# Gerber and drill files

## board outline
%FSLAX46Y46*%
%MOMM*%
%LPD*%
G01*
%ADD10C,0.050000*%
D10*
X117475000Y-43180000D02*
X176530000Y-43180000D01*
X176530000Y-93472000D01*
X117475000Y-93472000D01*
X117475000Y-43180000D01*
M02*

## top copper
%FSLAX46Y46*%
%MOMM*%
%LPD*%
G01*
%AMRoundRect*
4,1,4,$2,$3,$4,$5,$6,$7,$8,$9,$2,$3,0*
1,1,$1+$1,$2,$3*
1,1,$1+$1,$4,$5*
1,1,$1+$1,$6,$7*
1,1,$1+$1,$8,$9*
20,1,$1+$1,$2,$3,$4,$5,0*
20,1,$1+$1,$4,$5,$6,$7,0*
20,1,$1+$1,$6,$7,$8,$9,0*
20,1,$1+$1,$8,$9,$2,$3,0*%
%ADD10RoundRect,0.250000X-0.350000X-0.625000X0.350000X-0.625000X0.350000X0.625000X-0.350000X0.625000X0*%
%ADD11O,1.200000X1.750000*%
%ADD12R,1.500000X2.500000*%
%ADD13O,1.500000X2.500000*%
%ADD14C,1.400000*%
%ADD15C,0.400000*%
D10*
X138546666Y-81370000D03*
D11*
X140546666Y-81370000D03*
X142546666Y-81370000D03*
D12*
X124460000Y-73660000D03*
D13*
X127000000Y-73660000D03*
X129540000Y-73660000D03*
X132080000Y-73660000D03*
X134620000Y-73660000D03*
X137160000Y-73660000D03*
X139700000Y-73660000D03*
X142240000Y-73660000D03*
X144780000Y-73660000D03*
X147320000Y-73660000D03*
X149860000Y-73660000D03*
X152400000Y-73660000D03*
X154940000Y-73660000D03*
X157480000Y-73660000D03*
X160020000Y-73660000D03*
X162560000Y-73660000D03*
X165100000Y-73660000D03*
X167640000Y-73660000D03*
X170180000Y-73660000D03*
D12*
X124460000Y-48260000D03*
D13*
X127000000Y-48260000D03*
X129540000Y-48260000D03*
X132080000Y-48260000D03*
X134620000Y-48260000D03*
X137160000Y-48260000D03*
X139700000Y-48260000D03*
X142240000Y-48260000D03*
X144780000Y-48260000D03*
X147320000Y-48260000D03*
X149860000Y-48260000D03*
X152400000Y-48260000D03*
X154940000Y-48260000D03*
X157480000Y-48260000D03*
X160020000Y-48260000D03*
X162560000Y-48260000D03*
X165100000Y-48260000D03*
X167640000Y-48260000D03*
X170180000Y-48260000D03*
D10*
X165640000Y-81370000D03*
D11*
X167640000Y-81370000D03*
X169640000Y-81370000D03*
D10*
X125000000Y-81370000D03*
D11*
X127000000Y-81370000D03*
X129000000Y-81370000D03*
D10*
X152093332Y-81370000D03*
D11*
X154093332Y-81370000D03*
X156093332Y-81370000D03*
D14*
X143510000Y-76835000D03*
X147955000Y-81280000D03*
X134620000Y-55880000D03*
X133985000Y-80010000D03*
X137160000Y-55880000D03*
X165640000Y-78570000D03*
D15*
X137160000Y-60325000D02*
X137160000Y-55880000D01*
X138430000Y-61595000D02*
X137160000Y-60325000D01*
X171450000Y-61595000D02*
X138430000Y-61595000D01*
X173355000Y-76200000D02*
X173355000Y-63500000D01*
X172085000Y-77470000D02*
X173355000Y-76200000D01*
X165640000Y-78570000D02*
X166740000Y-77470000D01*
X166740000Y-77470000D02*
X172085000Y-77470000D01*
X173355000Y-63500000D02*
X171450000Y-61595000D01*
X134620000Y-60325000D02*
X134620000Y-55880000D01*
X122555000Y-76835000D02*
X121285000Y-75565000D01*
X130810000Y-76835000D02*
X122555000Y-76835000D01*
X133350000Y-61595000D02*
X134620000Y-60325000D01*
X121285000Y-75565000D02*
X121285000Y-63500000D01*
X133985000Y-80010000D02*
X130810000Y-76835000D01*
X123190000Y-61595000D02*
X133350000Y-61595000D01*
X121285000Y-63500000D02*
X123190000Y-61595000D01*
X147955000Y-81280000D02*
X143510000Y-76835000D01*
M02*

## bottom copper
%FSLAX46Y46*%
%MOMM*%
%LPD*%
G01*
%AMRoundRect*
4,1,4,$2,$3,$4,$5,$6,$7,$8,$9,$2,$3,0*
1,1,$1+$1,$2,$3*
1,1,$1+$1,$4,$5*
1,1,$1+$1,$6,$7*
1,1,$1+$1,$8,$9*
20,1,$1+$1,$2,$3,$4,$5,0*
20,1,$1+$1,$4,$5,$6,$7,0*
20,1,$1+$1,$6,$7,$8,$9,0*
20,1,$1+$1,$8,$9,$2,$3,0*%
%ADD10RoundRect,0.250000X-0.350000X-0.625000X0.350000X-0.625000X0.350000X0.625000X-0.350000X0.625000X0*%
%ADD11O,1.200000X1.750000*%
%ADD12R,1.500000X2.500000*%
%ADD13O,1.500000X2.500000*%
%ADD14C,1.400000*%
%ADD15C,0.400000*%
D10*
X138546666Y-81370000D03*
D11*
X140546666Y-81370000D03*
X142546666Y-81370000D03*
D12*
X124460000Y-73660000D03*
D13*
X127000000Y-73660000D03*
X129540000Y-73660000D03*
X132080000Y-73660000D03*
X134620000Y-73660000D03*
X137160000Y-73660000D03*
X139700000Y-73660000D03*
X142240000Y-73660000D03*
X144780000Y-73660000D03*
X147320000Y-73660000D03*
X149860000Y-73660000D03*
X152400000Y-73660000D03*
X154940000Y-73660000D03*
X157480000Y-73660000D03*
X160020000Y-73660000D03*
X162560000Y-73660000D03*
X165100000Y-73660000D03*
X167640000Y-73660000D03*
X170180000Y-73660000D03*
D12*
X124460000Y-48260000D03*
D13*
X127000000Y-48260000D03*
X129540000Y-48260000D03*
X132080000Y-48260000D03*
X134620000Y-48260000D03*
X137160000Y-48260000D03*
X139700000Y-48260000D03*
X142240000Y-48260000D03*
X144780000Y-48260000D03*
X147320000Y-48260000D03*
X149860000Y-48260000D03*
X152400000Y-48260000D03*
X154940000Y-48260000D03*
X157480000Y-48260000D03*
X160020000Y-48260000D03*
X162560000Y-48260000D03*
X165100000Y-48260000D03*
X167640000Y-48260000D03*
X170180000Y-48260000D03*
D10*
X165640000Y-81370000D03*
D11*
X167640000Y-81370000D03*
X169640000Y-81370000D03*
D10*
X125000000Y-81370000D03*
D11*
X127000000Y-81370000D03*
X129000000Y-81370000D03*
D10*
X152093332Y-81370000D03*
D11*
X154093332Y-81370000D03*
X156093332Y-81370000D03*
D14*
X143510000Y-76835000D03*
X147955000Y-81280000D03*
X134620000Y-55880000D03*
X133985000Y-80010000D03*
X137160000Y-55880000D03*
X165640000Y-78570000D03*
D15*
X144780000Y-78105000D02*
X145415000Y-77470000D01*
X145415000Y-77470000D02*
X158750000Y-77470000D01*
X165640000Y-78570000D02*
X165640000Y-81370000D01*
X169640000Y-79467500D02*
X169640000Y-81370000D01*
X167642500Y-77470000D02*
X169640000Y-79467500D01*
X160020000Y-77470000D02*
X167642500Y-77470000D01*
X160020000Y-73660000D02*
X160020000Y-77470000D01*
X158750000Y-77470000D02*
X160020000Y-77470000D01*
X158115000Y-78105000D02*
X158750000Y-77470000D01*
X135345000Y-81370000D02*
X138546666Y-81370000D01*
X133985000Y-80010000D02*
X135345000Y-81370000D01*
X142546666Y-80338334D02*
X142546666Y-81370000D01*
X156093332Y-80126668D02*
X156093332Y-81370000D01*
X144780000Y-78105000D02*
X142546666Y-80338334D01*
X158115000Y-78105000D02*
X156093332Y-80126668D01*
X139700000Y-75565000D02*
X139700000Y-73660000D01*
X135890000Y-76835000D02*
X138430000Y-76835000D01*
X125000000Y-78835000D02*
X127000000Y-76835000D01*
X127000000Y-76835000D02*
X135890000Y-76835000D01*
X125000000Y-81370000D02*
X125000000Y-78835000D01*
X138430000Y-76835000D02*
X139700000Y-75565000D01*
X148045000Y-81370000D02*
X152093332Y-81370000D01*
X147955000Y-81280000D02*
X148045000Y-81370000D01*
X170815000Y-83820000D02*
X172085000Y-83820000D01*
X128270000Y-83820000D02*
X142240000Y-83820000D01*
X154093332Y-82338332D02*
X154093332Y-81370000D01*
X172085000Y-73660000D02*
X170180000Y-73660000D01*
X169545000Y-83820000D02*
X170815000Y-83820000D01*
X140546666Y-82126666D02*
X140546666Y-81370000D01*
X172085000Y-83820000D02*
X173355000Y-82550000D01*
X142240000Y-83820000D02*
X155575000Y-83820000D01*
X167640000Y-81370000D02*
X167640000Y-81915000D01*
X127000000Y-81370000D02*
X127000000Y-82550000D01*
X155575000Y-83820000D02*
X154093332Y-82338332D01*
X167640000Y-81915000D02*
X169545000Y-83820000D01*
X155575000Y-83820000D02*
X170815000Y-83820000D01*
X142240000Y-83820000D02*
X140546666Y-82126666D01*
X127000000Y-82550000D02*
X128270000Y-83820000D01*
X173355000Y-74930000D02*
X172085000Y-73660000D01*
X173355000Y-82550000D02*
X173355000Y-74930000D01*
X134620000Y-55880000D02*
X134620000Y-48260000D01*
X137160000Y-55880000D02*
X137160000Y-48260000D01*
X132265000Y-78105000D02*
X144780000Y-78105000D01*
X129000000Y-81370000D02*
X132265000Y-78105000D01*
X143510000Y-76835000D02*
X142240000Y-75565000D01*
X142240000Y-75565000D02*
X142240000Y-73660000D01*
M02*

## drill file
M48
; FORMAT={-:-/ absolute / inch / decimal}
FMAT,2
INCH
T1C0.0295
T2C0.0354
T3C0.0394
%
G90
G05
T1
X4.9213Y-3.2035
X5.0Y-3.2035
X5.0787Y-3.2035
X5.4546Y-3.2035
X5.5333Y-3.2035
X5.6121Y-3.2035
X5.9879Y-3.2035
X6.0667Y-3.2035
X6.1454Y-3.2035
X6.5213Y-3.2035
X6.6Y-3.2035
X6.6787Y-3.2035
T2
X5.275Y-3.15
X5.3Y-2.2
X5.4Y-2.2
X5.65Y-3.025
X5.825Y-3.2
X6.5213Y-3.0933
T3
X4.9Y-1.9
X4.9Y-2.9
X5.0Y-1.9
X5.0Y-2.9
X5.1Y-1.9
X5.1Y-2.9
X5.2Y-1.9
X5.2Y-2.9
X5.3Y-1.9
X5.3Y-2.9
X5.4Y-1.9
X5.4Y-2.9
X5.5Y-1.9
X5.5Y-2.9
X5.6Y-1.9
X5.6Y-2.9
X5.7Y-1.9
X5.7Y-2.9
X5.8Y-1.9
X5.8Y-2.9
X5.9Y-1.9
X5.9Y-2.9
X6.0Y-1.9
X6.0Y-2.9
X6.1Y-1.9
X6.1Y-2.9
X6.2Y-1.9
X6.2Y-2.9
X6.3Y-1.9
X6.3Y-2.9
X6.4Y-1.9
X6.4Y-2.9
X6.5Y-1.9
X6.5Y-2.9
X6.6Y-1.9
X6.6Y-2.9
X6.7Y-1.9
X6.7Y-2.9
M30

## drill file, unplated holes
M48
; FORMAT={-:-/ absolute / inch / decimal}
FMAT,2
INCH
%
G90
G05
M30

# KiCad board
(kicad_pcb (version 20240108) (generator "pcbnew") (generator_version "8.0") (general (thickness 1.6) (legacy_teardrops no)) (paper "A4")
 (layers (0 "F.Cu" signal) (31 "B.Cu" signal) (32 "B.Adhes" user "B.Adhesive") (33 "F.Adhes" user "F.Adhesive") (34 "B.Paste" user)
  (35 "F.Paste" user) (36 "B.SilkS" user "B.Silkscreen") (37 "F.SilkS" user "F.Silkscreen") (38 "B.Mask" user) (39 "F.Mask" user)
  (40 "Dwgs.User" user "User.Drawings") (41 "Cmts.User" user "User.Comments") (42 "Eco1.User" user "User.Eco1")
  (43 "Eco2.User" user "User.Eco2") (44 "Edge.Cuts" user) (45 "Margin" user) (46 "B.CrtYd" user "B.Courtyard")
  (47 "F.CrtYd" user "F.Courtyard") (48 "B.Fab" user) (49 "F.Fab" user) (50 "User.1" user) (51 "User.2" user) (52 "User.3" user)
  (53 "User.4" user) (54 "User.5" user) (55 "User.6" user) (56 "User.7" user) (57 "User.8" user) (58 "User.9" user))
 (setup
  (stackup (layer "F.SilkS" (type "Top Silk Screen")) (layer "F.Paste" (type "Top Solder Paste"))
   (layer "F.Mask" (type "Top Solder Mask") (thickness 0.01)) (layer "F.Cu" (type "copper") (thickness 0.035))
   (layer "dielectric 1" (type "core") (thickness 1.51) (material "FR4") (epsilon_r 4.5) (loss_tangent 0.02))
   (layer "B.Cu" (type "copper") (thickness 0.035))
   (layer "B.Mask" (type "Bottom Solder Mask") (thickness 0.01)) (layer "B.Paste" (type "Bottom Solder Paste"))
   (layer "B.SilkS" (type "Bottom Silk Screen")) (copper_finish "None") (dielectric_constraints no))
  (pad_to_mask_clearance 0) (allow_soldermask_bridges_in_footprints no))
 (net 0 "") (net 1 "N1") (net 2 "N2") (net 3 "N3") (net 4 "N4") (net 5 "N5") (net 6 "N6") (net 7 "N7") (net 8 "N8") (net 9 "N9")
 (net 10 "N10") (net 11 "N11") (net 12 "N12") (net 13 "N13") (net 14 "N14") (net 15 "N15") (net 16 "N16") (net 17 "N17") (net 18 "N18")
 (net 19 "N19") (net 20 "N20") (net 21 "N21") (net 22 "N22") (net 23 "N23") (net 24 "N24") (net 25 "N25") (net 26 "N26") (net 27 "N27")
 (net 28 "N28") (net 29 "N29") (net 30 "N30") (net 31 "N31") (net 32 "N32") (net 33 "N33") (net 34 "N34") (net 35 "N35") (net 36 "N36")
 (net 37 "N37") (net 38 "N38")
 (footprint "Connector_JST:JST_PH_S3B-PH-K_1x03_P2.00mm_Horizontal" (layer "F.Cu") (at 138.546666 81.37)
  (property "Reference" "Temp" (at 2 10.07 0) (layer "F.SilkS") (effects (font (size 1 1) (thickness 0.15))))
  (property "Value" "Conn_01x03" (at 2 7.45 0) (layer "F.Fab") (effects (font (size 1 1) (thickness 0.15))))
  (pad "1" thru_hole roundrect (at 0 0) (size 1.2 1.75) (drill 0.75) (layers "*.Cu" "*.Mask") (remove_unused_layers no)
   (roundrect_rratio 0.208333) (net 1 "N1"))
  (pad "2" thru_hole oval (at 2 0) (size 1.2 1.75) (drill 0.75) (layers "*.Cu" "*.Mask") (remove_unused_layers no) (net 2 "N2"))
  (pad "3" thru_hole oval (at 4 0) (size 1.2 1.75) (drill 0.75) (layers "*.Cu" "*.Mask") (remove_unused_layers no) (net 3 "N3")))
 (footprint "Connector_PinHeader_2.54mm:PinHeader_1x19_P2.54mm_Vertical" (layer "F.Cu") (at 124.46 73.66 90)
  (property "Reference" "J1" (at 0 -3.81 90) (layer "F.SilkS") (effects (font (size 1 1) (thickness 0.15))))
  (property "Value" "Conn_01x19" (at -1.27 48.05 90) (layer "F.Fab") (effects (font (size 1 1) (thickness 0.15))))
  (pad "1" thru_hole rect (at 0 0 90) (size 2.5 1.5) (drill 1) (layers "*.Cu" "*.Mask") (remove_unused_layers no) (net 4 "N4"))
  (pad "2" thru_hole oval (at 0 2.54 90) (size 2.5 1.5) (drill 1) (layers "*.Cu" "*.Mask") (remove_unused_layers no) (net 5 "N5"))
  (pad "3" thru_hole oval (at 0 5.08 90) (size 2.5 1.5) (drill 1) (layers "*.Cu" "*.Mask") (remove_unused_layers no) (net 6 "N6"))
  (pad "4" thru_hole oval (at 0 7.62 90) (size 2.5 1.5) (drill 1) (layers "*.Cu" "*.Mask") (remove_unused_layers no) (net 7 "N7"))
  (pad "5" thru_hole oval (at 0 10.16 90) (size 2.5 1.5) (drill 1) (layers "*.Cu" "*.Mask") (remove_unused_layers no) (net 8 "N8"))
  (pad "6" thru_hole oval (at 0 12.7 90) (size 2.5 1.5) (drill 1) (layers "*.Cu" "*.Mask") (remove_unused_layers no) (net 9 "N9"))
  (pad "7" thru_hole oval (at 0 15.24 90) (size 2.5 1.5) (drill 1) (layers "*.Cu" "*.Mask") (remove_unused_layers no) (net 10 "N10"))
  (pad "8" thru_hole oval (at 0 17.78 90) (size 2.5 1.5) (drill 1) (layers "*.Cu" "*.Mask") (remove_unused_layers no) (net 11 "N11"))
  (pad "9" thru_hole oval (at 0 20.32 90) (size 2.5 1.5) (drill 1) (layers "*.Cu" "*.Mask") (remove_unused_layers no) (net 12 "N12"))
  (pad "10" thru_hole oval (at 0 22.86 90) (size 2.5 1.5) (drill 1) (layers "*.Cu" "*.Mask") (remove_unused_layers no) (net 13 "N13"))
  (pad "11" thru_hole oval (at 0 25.4 90) (size 2.5 1.5) (drill 1) (layers "*.Cu" "*.Mask") (remove_unused_layers no) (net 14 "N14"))
  (pad "12" thru_hole oval (at 0 27.94 90) (size 2.5 1.5) (drill 1) (layers "*.Cu" "*.Mask") (remove_unused_layers no) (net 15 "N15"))
  (pad "13" thru_hole oval (at 0 30.48 90) (size 2.5 1.5) (drill 1) (layers "*.Cu" "*.Mask") (remove_unused_layers no) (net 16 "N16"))
  (pad "14" thru_hole oval (at 0 33.02 90) (size 2.5 1.5) (drill 1) (layers "*.Cu" "*.Mask") (remove_unused_layers no) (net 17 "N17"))
  (pad "15" thru_hole oval (at 0 35.56 90) (size 2.5 1.5) (drill 1) (layers "*.Cu" "*.Mask") (remove_unused_layers no) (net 3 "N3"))
  (pad "16" thru_hole oval (at 0 38.1 90) (size 2.5 1.5) (drill 1) (layers "*.Cu" "*.Mask") (remove_unused_layers no) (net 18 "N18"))
  (pad "17" thru_hole oval (at 0 40.64 90) (size 2.5 1.5) (drill 1) (layers "*.Cu" "*.Mask") (remove_unused_layers no) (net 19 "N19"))
  (pad "18" thru_hole oval (at 0 43.18 90) (size 2.5 1.5) (drill 1) (layers "*.Cu" "*.Mask") (remove_unused_layers no) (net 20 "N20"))
  (pad "19" thru_hole oval (at 0 45.72 90) (size 2.5 1.5) (drill 1) (layers "*.Cu" "*.Mask") (remove_unused_layers no) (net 2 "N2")))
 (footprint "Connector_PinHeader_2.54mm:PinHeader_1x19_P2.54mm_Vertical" (layer "F.Cu") (at 124.46 48.26 90)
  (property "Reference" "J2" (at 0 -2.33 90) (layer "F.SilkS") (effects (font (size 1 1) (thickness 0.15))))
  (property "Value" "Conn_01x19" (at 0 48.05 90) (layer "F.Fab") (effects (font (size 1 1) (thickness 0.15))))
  (pad "1" thru_hole rect (at 0 0 90) (size 2.5 1.5) (drill 1) (layers "*.Cu" "*.Mask") (remove_unused_layers no) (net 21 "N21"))
  (pad "2" thru_hole oval (at 0 2.54 90) (size 2.5 1.5) (drill 1) (layers "*.Cu" "*.Mask") (remove_unused_layers no) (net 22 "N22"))
  (pad "3" thru_hole oval (at 0 5.08 90) (size 2.5 1.5) (drill 1) (layers "*.Cu" "*.Mask") (remove_unused_layers no) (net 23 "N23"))
  (pad "4" thru_hole oval (at 0 7.62 90) (size 2.5 1.5) (drill 1) (layers "*.Cu" "*.Mask") (remove_unused_layers no) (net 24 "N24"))
  (pad "5" thru_hole oval (at 0 10.16 90) (size 2.5 1.5) (drill 1) (layers "*.Cu" "*.Mask") (remove_unused_layers no) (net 1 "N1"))
  (pad "6" thru_hole oval (at 0 12.7 90) (size 2.5 1.5) (drill 1) (layers "*.Cu" "*.Mask") (remove_unused_layers no) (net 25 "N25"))
  (pad "7" thru_hole oval (at 0 15.24 90) (size 2.5 1.5) (drill 1) (layers "*.Cu" "*.Mask") (remove_unused_layers no) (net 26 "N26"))
  (pad "8" thru_hole oval (at 0 17.78 90) (size 2.5 1.5) (drill 1) (layers "*.Cu" "*.Mask") (remove_unused_layers no) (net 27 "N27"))
  (pad "9" thru_hole oval (at 0 20.32 90) (size 2.5 1.5) (drill 1) (layers "*.Cu" "*.Mask") (remove_unused_layers no) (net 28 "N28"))
  (pad "10" thru_hole oval (at 0 22.86 90) (size 2.5 1.5) (drill 1) (layers "*.Cu" "*.Mask") (remove_unused_layers no) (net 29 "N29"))
  (pad "11" thru_hole oval (at 0 25.4 90) (size 2.5 1.5) (drill 1) (layers "*.Cu" "*.Mask") (remove_unused_layers no) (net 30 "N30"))
  (pad "12" thru_hole oval (at 0 27.94 90) (size 2.5 1.5) (drill 1) (layers "*.Cu" "*.Mask") (remove_unused_layers no) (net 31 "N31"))
  (pad "13" thru_hole oval (at 0 30.48 90) (size 2.5 1.5) (drill 1) (layers "*.Cu" "*.Mask") (remove_unused_layers no) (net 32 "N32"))
  (pad "14" thru_hole oval (at 0 33.02 90) (size 2.5 1.5) (drill 1) (layers "*.Cu" "*.Mask") (remove_unused_layers no) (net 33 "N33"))
  (pad "15" thru_hole oval (at 0 35.56 90) (size 2.5 1.5) (drill 1) (layers "*.Cu" "*.Mask") (remove_unused_layers no) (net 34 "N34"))
  (pad "16" thru_hole oval (at 0 38.1 90) (size 2.5 1.5) (drill 1) (layers "*.Cu" "*.Mask") (remove_unused_layers no) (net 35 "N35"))
  (pad "17" thru_hole oval (at 0 40.64 90) (size 2.5 1.5) (drill 1) (layers "*.Cu" "*.Mask") (remove_unused_layers no) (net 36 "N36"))
  (pad "18" thru_hole oval (at 0 43.18 90) (size 2.5 1.5) (drill 1) (layers "*.Cu" "*.Mask") (remove_unused_layers no) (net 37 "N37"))
  (pad "19" thru_hole oval (at 0 45.72 90) (size 2.5 1.5) (drill 1) (layers "*.Cu" "*.Mask") (remove_unused_layers no) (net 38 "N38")))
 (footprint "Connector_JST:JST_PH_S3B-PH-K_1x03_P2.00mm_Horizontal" (layer "F.Cu") (at 165.64 81.37)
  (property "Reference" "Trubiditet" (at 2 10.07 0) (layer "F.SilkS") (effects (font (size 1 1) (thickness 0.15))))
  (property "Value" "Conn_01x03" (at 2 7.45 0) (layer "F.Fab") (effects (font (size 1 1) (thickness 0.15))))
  (pad "1" thru_hole roundrect (at 0 0) (size 1.2 1.75) (drill 0.75) (layers "*.Cu" "*.Mask") (remove_unused_layers no)
   (roundrect_rratio 0.208333) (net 25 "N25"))
  (pad "2" thru_hole oval (at 2 0) (size 1.2 1.75) (drill 0.75) (layers "*.Cu" "*.Mask") (remove_unused_layers no) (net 2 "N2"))
  (pad "3" thru_hole oval (at 4 0) (size 1.2 1.75) (drill 0.75) (layers "*.Cu" "*.Mask") (remove_unused_layers no) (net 3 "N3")))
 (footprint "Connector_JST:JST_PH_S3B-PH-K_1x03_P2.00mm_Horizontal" (layer "F.Cu") (at 125 81.37)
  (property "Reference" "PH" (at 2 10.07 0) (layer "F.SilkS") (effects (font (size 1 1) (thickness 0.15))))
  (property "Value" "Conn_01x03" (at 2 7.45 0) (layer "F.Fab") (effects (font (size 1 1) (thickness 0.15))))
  (pad "1" thru_hole roundrect (at 0 0) (size 1.2 1.75) (drill 0.75) (layers "*.Cu" "*.Mask") (remove_unused_layers no)
   (roundrect_rratio 0.208333) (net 10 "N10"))
  (pad "2" thru_hole oval (at 2 0) (size 1.2 1.75) (drill 0.75) (layers "*.Cu" "*.Mask") (remove_unused_layers no) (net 2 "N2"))
  (pad "3" thru_hole oval (at 4 0) (size 1.2 1.75) (drill 0.75) (layers "*.Cu" "*.Mask") (remove_unused_layers no) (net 3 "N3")))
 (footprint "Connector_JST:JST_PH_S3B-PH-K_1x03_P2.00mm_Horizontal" (layer "F.Cu") (at 152.093332 81.37)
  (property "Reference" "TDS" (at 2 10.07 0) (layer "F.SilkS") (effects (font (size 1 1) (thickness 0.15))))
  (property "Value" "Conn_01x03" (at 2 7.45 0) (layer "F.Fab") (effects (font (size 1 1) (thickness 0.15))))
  (pad "1" thru_hole roundrect (at 0 0) (size 1.2 1.75) (drill 0.75) (layers "*.Cu" "*.Mask") (remove_unused_layers no)
   (roundrect_rratio 0.208333) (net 11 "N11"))
  (pad "2" thru_hole oval (at 2 0) (size 1.2 1.75) (drill 0.75) (layers "*.Cu" "*.Mask") (remove_unused_layers no) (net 2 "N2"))
  (pad "3" thru_hole oval (at 4 0) (size 1.2 1.75) (drill 0.75) (layers "*.Cu" "*.Mask") (remove_unused_layers no) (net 3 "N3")))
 (gr_rect (start 117.475 43.18) (end 176.53 93.472) (stroke (width 0.05) (type default)) (fill none) (layer "Edge.Cuts"))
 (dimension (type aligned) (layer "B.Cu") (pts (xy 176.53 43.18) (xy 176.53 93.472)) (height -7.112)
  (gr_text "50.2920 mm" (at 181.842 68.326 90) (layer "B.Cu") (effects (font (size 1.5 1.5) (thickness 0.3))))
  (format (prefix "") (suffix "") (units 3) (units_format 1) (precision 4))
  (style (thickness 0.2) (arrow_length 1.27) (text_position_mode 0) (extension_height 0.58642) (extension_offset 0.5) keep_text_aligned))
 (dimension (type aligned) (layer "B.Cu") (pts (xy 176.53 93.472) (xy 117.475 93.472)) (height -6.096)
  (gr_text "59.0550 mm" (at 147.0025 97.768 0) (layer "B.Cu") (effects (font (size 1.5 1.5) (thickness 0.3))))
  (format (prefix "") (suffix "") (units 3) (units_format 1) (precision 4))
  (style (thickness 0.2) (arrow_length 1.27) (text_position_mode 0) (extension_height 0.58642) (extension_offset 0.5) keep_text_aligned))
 (segment (start 160.02 73.66) (end 160.02 77.47) (width 0.4) (layer "B.Cu") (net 3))
 (segment (start 142.546666 80.338334) (end 142.546666 81.37) (width 0.4) (layer "B.Cu") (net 3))
 (segment (start 156.093332 80.126668) (end 156.093332 81.37) (width 0.4) (layer "B.Cu") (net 3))
 (segment (start 167.6425 77.47) (end 169.64 79.4675) (width 0.4) (layer "B.Cu") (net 3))
 (segment (start 169.64 79.4675) (end 169.64 81.37) (width 0.4) (layer "B.Cu") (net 3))
 (segment (start 158.75 77.47) (end 160.02 77.47) (width 0.4) (layer "B.Cu") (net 3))
 (segment (start 144.78 78.105) (end 145.415 77.47) (width 0.4) (layer "B.Cu") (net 3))
 (segment (start 144.78 78.105) (end 142.546666 80.338334) (width 0.4) (layer "B.Cu") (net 3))
 (segment (start 158.115 78.105) (end 158.75 77.47) (width 0.4) (layer "B.Cu") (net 3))
 (segment (start 129 81.37) (end 132.265 78.105) (width 0.4) (layer "B.Cu") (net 3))
 (segment (start 158.115 78.105) (end 156.093332 80.126668) (width 0.4) (layer "B.Cu") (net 3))
 (segment (start 160.02 77.47) (end 167.6425 77.47) (width 0.4) (layer "B.Cu") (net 3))
 (segment (start 145.415 77.47) (end 158.75 77.47) (width 0.4) (layer "B.Cu") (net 3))
 (segment (start 132.265 78.105) (end 144.78 78.105) (width 0.4) (layer "B.Cu") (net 3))
 (segment (start 139.7 75.565) (end 139.7 73.66) (width 0.4) (layer "B.Cu") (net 10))
 (segment (start 135.89 76.835) (end 138.43 76.835) (width 0.4) (layer "B.Cu") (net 10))
 (segment (start 125 78.835) (end 127 76.835) (width 0.4) (layer "B.Cu") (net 10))
 (segment (start 127 76.835) (end 135.89 76.835) (width 0.4) (layer "B.Cu") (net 10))
 (segment (start 125 81.37) (end 125 78.835) (width 0.4) (layer "B.Cu") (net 10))
 (segment (start 138.43 76.835) (end 139.7 75.565) (width 0.4) (layer "B.Cu") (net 10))
 (segment (start 147.955 81.28) (end 143.51 76.835) (width 0.4) (layer "F.Cu") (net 11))
 (via (at 143.51 76.835) (size 1.4) (drill 0.9) (layers "F.Cu" "B.Cu") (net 11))
 (via (at 147.955 81.28) (size 1.4) (drill 0.9) (layers "F.Cu" "B.Cu") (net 11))
 (segment (start 148.045 81.37) (end 152.093332 81.37) (width 0.4) (layer "B.Cu") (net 11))
 (segment (start 143.51 76.835) (end 142.24 75.565) (width 0.4) (layer "B.Cu") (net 11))
 (segment (start 147.955 81.28) (end 148.045 81.37) (width 0.4) (layer "B.Cu") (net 11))
 (segment (start 142.24 75.565) (end 142.24 73.66) (width 0.4) (layer "B.Cu") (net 11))
 (segment (start 170.815 83.82) (end 172.085 83.82) (width 0.4) (layer "B.Cu") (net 2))
 (segment (start 128.27 83.82) (end 142.24 83.82) (width 0.4) (layer "B.Cu") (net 2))
 (segment (start 154.093332 82.338332) (end 154.093332 81.37) (width 0.4) (layer "B.Cu") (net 2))
 (segment (start 172.085 73.66) (end 170.18 73.66) (width 0.4) (layer "B.Cu") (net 2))
 (segment (start 169.545 83.82) (end 170.815 83.82) (width 0.4) (layer "B.Cu") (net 2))
 (segment (start 140.546666 82.126666) (end 140.546666 81.37) (width 0.4) (layer "B.Cu") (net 2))
 (segment (start 172.085 83.82) (end 173.355 82.55) (width 0.4) (layer "B.Cu") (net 2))
 (segment (start 142.24 83.82) (end 155.575 83.82) (width 0.4) (layer "B.Cu") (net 2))
 (segment (start 167.64 81.37) (end 167.64 81.915) (width 0.4) (layer "B.Cu") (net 2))
 (segment (start 127 81.37) (end 127 82.55) (width 0.4) (layer "B.Cu") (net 2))
 (segment (start 155.575 83.82) (end 154.093332 82.338332) (width 0.4) (layer "B.Cu") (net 2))
 (segment (start 167.64 81.915) (end 169.545 83.82) (width 0.4) (layer "B.Cu") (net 2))
 (segment (start 155.575 83.82) (end 170.815 83.82) (width 0.4) (layer "B.Cu") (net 2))
 (segment (start 142.24 83.82) (end 140.546666 82.126666) (width 0.4) (layer "B.Cu") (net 2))
 (segment (start 127 82.55) (end 128.27 83.82) (width 0.4) (layer "B.Cu") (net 2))
 (segment (start 173.355 74.93) (end 172.085 73.66) (width 0.4) (layer "B.Cu") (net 2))
 (segment (start 173.355 82.55) (end 173.355 74.93) (width 0.4) (layer "B.Cu") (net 2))
 (segment (start 123.19 61.595) (end 133.35 61.595) (width 0.4) (layer "F.Cu") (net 1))
 (segment (start 133.35 61.595) (end 134.62 60.325) (width 0.4) (layer "F.Cu") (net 1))
 (segment (start 121.285 75.565) (end 121.285 63.5) (width 0.4) (layer "F.Cu") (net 1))
 (segment (start 130.81 76.835) (end 122.555 76.835) (width 0.4) (layer "F.Cu") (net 1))
 (segment (start 133.985 80.01) (end 130.81 76.835) (width 0.4) (layer "F.Cu") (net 1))
 (segment (start 134.62 60.325) (end 134.62 55.88) (width 0.4) (layer "F.Cu") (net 1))
 (segment (start 122.555 76.835) (end 121.285 75.565) (width 0.4) (layer "F.Cu") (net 1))
 (segment (start 121.285 63.5) (end 123.19 61.595) (width 0.4) (layer "F.Cu") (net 1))
 (via (at 134.62 55.88) (size 1.4) (drill 0.9) (layers "F.Cu" "B.Cu") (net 1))
 (via (at 133.985 80.01) (size 1.4) (drill 0.9) (layers "F.Cu" "B.Cu") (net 1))
 (segment (start 135.345 81.37) (end 138.546666 81.37) (width 0.4) (layer "B.Cu") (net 1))
 (segment (start 134.62 55.88) (end 134.62 48.26) (width 0.4) (layer "B.Cu") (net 1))
 (segment (start 133.985 80.01) (end 135.345 81.37) (width 0.4) (layer "B.Cu") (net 1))
 (segment (start 166.74 77.47) (end 172.085 77.47) (width 0.4) (layer "F.Cu") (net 25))
 (segment (start 165.64 78.57) (end 166.74 77.47) (width 0.4) (layer "F.Cu") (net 25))
 (segment (start 173.355 76.2) (end 173.355 63.5) (width 0.4) (layer "F.Cu") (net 25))
 (segment (start 173.355 63.5) (end 171.45 61.595) (width 0.4) (layer "F.Cu") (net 25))
 (segment (start 171.45 61.595) (end 138.43 61.595) (width 0.4) (layer "F.Cu") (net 25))
 (segment (start 137.16 60.325) (end 137.16 55.88) (width 0.4) (layer "F.Cu") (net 25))
 (segment (start 138.43 61.595) (end 137.16 60.325) (width 0.4) (layer "F.Cu") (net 25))
 (segment (start 172.085 77.47) (end 173.355 76.2) (width 0.4) (layer "F.Cu") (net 25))
 (via (at 137.16 55.88) (size 1.4) (drill 0.9) (layers "F.Cu" "B.Cu") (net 25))
 (via (at 165.64 78.57) (size 1.4) (drill 0.9) (layers "F.Cu" "B.Cu") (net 25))
 (segment (start 137.16 55.88) (end 137.16 48.26) (width 0.4) (layer "B.Cu") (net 25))
 (segment (start 165.64 78.57) (end 165.64 81.37) (width 0.4) (layer "B.Cu") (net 25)))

